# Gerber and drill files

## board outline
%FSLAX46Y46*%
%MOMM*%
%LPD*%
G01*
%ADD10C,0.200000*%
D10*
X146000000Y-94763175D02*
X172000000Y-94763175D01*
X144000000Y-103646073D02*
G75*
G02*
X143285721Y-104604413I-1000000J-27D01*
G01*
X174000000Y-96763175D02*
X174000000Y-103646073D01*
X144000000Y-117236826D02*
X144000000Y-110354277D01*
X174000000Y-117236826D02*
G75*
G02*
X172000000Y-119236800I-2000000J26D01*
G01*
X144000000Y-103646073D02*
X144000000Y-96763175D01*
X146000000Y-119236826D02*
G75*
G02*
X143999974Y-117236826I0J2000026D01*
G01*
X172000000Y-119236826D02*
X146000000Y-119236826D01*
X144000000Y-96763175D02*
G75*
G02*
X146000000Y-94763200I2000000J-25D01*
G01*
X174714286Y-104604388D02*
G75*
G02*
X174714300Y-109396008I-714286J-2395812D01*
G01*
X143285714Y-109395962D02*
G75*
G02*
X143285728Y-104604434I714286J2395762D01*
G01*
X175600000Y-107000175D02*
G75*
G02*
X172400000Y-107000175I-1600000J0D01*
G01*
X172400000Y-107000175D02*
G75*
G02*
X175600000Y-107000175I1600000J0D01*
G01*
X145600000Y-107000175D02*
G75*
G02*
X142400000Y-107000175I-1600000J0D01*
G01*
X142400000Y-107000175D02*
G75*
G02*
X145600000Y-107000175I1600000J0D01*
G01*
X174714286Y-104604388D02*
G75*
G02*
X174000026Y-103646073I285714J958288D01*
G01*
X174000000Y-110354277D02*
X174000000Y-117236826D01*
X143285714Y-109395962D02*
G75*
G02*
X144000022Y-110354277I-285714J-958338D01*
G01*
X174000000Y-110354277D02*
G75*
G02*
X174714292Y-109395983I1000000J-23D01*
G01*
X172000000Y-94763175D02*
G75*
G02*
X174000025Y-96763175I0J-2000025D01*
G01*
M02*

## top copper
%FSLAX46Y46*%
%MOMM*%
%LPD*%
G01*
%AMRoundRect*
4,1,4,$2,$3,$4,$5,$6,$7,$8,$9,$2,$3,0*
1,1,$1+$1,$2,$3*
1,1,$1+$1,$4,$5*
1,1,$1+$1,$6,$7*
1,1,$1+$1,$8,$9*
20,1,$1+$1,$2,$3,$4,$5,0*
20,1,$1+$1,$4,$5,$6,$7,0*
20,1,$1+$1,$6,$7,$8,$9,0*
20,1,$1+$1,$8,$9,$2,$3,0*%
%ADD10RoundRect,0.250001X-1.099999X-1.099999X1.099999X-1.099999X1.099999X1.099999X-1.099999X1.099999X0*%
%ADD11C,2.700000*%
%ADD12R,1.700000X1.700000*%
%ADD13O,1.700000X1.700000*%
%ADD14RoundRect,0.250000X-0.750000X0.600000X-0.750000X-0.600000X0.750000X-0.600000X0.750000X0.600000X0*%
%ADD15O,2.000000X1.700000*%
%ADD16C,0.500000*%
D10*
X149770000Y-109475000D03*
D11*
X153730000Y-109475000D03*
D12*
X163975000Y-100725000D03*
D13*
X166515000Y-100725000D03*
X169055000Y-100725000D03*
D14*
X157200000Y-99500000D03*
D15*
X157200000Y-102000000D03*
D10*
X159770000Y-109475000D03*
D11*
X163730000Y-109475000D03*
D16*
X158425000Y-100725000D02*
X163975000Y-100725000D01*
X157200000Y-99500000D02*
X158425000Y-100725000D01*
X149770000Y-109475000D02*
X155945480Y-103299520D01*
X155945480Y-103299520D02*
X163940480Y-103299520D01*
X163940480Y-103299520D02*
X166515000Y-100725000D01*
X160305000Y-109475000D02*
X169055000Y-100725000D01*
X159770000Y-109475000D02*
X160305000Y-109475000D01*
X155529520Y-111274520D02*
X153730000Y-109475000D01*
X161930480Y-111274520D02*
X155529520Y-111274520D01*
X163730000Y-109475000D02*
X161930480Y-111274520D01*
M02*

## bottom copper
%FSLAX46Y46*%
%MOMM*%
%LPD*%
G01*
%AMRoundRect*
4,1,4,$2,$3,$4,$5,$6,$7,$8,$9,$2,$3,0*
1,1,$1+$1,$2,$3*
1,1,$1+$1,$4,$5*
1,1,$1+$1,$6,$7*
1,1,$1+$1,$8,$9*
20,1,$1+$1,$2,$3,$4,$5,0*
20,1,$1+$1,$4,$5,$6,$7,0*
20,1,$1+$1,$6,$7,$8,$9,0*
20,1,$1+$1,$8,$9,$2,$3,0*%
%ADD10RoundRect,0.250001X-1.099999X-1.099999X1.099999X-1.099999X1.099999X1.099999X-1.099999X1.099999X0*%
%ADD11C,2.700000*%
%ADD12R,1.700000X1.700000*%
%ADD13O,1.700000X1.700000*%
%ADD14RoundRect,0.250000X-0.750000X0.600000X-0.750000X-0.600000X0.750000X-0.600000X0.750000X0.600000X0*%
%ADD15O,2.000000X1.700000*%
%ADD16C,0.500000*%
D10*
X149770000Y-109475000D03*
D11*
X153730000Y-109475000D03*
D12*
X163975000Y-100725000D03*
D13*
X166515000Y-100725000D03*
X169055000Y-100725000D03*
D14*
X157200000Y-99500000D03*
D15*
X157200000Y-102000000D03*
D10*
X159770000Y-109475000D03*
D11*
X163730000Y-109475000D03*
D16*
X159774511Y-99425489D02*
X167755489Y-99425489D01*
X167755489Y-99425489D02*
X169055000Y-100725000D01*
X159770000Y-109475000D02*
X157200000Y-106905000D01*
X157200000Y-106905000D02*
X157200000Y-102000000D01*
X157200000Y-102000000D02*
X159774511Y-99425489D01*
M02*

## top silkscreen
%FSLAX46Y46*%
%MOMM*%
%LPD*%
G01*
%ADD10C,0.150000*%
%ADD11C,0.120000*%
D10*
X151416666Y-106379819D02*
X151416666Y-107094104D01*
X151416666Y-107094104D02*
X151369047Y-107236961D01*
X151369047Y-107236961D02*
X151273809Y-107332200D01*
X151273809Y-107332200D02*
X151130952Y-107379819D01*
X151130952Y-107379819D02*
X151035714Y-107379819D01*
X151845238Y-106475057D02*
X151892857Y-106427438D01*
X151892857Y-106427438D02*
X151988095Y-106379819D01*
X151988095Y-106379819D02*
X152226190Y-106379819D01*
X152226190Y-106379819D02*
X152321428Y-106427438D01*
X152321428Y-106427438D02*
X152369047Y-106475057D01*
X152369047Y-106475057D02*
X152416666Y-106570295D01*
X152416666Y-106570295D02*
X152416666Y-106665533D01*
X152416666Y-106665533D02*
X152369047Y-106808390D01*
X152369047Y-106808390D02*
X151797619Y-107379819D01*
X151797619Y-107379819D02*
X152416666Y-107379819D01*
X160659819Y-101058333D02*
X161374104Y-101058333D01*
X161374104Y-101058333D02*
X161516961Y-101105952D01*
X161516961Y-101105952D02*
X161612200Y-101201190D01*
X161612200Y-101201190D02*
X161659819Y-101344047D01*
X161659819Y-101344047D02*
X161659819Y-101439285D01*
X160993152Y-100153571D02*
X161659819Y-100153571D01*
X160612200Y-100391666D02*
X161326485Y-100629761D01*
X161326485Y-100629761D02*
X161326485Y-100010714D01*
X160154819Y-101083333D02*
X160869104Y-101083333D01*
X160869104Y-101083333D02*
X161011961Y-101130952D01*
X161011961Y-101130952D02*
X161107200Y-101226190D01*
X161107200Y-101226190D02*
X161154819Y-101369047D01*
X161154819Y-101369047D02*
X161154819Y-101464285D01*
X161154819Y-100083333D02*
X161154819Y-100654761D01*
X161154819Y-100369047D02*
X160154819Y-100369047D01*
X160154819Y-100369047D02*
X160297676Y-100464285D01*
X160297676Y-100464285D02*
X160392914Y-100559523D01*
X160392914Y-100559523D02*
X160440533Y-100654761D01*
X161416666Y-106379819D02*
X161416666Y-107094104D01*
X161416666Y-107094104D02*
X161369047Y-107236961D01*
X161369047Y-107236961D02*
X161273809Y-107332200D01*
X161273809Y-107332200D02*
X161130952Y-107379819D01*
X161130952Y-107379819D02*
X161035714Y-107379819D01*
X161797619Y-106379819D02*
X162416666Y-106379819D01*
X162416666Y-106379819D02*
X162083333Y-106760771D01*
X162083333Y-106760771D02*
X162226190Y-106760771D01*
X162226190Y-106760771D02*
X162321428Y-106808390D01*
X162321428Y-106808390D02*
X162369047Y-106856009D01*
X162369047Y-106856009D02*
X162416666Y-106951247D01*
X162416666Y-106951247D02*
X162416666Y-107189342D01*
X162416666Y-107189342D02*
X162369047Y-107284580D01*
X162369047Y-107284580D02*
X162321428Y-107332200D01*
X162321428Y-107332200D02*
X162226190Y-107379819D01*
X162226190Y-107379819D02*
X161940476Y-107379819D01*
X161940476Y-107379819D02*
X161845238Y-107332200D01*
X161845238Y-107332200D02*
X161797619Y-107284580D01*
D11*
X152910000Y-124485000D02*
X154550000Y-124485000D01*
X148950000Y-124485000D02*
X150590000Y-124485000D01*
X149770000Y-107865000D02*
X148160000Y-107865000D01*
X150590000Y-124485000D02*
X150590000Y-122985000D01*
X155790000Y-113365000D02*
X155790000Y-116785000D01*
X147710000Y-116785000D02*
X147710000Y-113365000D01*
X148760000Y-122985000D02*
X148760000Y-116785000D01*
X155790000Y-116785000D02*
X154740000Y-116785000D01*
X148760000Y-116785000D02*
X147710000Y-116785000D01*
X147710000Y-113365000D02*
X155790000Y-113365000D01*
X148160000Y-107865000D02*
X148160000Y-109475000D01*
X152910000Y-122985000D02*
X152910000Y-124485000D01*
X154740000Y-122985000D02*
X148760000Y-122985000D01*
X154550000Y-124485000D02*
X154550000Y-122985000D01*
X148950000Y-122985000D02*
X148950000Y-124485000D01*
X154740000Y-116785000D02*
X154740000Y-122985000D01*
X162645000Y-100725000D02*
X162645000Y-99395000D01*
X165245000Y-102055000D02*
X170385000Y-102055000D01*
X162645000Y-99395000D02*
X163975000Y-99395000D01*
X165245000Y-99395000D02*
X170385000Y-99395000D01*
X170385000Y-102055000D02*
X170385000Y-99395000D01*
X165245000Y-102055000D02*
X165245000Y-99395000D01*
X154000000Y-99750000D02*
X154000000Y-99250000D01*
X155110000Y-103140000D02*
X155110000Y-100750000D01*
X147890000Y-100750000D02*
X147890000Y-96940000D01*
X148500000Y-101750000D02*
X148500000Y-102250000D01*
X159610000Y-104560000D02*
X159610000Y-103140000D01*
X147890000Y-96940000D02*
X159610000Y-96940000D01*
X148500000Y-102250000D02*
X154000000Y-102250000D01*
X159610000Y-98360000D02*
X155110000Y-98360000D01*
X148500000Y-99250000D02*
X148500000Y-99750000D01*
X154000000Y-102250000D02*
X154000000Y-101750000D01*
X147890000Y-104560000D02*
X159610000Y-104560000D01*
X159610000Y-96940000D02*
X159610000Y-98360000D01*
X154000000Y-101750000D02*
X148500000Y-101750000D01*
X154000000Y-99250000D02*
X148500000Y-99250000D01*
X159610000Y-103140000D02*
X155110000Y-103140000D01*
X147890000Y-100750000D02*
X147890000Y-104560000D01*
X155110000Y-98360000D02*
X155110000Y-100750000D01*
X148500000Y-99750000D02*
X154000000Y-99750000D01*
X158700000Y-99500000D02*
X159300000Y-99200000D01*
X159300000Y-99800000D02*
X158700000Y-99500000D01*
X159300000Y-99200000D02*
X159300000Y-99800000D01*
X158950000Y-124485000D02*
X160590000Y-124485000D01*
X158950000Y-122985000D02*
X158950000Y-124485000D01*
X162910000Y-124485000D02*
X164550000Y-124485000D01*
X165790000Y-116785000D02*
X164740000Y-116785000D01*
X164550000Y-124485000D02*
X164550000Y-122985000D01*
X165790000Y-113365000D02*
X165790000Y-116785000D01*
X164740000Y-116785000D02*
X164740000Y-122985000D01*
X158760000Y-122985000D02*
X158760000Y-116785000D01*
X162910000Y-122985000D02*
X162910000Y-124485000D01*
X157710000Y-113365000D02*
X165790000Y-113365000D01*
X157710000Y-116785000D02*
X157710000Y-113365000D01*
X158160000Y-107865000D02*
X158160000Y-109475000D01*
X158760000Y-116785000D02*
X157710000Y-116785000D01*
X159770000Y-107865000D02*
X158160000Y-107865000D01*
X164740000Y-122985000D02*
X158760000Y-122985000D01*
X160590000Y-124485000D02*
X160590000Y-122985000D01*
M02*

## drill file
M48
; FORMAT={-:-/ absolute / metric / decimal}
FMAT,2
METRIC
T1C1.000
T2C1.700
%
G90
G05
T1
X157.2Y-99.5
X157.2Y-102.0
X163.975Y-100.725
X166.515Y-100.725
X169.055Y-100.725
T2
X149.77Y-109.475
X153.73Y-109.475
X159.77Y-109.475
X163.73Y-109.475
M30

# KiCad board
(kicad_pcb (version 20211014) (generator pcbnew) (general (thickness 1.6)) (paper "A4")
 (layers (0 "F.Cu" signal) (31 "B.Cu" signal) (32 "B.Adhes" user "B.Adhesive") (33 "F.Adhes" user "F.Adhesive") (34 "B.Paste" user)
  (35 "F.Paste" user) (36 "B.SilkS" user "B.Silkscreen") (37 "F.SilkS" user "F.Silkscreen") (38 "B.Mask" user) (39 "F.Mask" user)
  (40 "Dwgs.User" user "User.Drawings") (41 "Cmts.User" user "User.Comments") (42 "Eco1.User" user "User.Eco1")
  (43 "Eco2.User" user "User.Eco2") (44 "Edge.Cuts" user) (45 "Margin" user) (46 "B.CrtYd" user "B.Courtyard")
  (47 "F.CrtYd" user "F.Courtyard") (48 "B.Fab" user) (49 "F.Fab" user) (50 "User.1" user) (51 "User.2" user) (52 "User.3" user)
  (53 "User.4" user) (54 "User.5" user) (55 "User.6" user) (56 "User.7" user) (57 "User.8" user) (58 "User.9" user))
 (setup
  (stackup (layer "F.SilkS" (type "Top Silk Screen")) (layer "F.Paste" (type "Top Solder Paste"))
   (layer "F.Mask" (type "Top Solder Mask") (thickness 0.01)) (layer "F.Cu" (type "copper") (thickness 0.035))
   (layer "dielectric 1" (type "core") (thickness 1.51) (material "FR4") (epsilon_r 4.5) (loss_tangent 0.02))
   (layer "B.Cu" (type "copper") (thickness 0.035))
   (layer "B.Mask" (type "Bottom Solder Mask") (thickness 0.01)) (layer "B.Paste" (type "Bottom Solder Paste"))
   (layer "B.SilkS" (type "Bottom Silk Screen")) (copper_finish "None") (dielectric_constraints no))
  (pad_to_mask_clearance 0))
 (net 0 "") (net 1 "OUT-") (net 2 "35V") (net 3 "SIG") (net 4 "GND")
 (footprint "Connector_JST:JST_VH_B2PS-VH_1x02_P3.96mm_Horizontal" (layer "F.Cu") (at 149.77 109.475)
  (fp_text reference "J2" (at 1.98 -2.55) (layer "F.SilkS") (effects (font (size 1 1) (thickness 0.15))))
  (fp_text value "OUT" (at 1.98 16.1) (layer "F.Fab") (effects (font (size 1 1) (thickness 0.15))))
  (fp_line (start 3.14 15.01) (end 4.78 15.01) (layer "F.SilkS") (width 0.12))
  (fp_line (start -0.82 15.01) (end 0.82 15.01) (layer "F.SilkS") (width 0.12))
  (fp_line (start 0 -1.61) (end -1.61 -1.61) (layer "F.SilkS") (width 0.12))
  (fp_line (start 0.82 15.01) (end 0.82 13.51) (layer "F.SilkS") (width 0.12))
  (fp_line (start 6.02 3.89) (end 6.02 7.31) (layer "F.SilkS") (width 0.12))
  (fp_line (start -2.06 7.31) (end -2.06 3.89) (layer "F.SilkS") (width 0.12))
  (fp_line (start -1.01 13.51) (end -1.01 7.31) (layer "F.SilkS") (width 0.12))
  (fp_line (start 6.02 7.31) (end 4.97 7.31) (layer "F.SilkS") (width 0.12))
  (fp_line (start -1.01 7.31) (end -2.06 7.31) (layer "F.SilkS") (width 0.12))
  (fp_line (start -2.06 3.89) (end 6.02 3.89) (layer "F.SilkS") (width 0.12))
  (fp_line (start -1.61 -1.61) (end -1.61 0) (layer "F.SilkS") (width 0.12))
  (fp_line (start 3.14 13.51) (end 3.14 15.01) (layer "F.SilkS") (width 0.12))
  (fp_line (start 4.97 13.51) (end -1.01 13.51) (layer "F.SilkS") (width 0.12))
  (fp_line (start 4.78 15.01) (end 4.78 13.51) (layer "F.SilkS") (width 0.12))
  (fp_line (start -0.82 13.51) (end -0.82 15.01) (layer "F.SilkS") (width 0.12))
  (fp_line (start 4.97 7.31) (end 4.97 13.51) (layer "F.SilkS") (width 0.12))
  (pad "1" thru_hole roundrect (at 0 0) (size 2.7 2.7) (drill 1.7) (layers *.Cu *.Mask) (roundrect_rratio 0.09259296296) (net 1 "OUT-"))
  (pad "2" thru_hole circle (at 3.96 0) (size 2.7 2.7) (drill 1.7) (layers *.Cu *.Mask) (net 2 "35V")))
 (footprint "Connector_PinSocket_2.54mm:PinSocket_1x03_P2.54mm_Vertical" (layer "F.Cu") (at 163.975 100.725 90)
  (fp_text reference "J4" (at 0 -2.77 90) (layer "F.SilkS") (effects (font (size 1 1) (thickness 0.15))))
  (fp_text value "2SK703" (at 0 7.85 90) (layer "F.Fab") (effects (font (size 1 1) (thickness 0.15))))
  (fp_line (start 0 -1.33) (end 1.33 -1.33) (layer "F.SilkS") (width 0.12))
  (fp_line (start -1.33 1.27) (end -1.33 6.41) (layer "F.SilkS") (width 0.12))
  (fp_line (start 1.33 -1.33) (end 1.33 0) (layer "F.SilkS") (width 0.12))
  (fp_line (start 1.33 1.27) (end 1.33 6.41) (layer "F.SilkS") (width 0.12))
  (fp_line (start -1.33 6.41) (end 1.33 6.41) (layer "F.SilkS") (width 0.12))
  (fp_line (start -1.33 1.27) (end 1.33 1.27) (layer "F.SilkS") (width 0.12))
  (pad "1" thru_hole rect (at 0 0 90) (size 1.7 1.7) (drill 1) (layers *.Cu *.Mask) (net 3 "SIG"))
  (pad "2" thru_hole oval (at 0 2.54 90) (size 1.7 1.7) (drill 1) (layers *.Cu *.Mask) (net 1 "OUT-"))
  (pad "3" thru_hole oval (at 0 5.08 90) (size 1.7 1.7) (drill 1) (layers *.Cu *.Mask) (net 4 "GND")))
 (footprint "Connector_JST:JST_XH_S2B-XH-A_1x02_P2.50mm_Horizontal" (layer "F.Cu") (at 157.2 99.5 -90)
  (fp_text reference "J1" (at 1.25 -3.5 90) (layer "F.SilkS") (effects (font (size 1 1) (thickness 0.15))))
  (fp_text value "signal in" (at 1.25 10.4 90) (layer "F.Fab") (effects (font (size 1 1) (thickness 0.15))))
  (fp_line (start 0.25 3.2) (end -0.25 3.2) (layer "F.SilkS") (width 0.12))
  (fp_line (start 3.64 2.09) (end 1.25 2.09) (layer "F.SilkS") (width 0.12))
  (fp_line (start 1.25 9.31) (end -2.56 9.31) (layer "F.SilkS") (width 0.12))
  (fp_line (start 2.25 8.7) (end 2.75 8.7) (layer "F.SilkS") (width 0.12))
  (fp_line (start 5.06 -2.41) (end 3.64 -2.41) (layer "F.SilkS") (width 0.12))
  (fp_line (start -2.56 9.31) (end -2.56 -2.41) (layer "F.SilkS") (width 0.12))
  (fp_line (start 2.75 8.7) (end 2.75 3.2) (layer "F.SilkS") (width 0.12))
  (fp_line (start -1.14 -2.41) (end -1.14 2.09) (layer "F.SilkS") (width 0.12))
  (fp_line (start -0.25 8.7) (end 0.25 8.7) (layer "F.SilkS") (width 0.12))
  (fp_line (start 2.75 3.2) (end 2.25 3.2) (layer "F.SilkS") (width 0.12))
  (fp_line (start 5.06 9.31) (end 5.06 -2.41) (layer "F.SilkS") (width 0.12))
  (fp_line (start -2.56 -2.41) (end -1.14 -2.41) (layer "F.SilkS") (width 0.12))
  (fp_line (start 2.25 3.2) (end 2.25 8.7) (layer "F.SilkS") (width 0.12))
  (fp_line (start -0.25 3.2) (end -0.25 8.7) (layer "F.SilkS") (width 0.12))
  (fp_line (start 3.64 -2.41) (end 3.64 2.09) (layer "F.SilkS") (width 0.12))
  (fp_line (start 1.25 9.31) (end 5.06 9.31) (layer "F.SilkS") (width 0.12))
  (fp_line (start -1.14 2.09) (end 1.25 2.09) (layer "F.SilkS") (width 0.12))
  (fp_line (start 0.25 8.7) (end 0.25 3.2) (layer "F.SilkS") (width 0.12))
  (fp_line (start 0 -1.5) (end -0.3 -2.1) (layer "F.SilkS") (width 0.12))
  (fp_line (start 0.3 -2.1) (end 0 -1.5) (layer "F.SilkS") (width 0.12))
  (fp_line (start -0.3 -2.1) (end 0.3 -2.1) (layer "F.SilkS") (width 0.12))
  (pad "1" thru_hole roundrect (at 0 0 270) (size 1.7 2) (drill 1) (layers *.Cu *.Mask) (roundrect_rratio 0.1470588235) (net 3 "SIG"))
  (pad "2" thru_hole oval (at 2.5 0 270) (size 1.7 2) (drill 1) (layers *.Cu *.Mask) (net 4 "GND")))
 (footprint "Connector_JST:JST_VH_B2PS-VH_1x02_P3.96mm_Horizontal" (layer "F.Cu") (at 159.77 109.475)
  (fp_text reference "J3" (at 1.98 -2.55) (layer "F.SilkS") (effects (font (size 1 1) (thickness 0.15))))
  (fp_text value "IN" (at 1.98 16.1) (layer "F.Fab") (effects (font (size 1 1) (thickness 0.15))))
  (fp_line (start -0.82 15.01) (end 0.82 15.01) (layer "F.SilkS") (width 0.12))
  (fp_line (start -0.82 13.51) (end -0.82 15.01) (layer "F.SilkS") (width 0.12))
  (fp_line (start 3.14 15.01) (end 4.78 15.01) (layer "F.SilkS") (width 0.12))
  (fp_line (start 6.02 7.31) (end 4.97 7.31) (layer "F.SilkS") (width 0.12))
  (fp_line (start 4.78 15.01) (end 4.78 13.51) (layer "F.SilkS") (width 0.12))
  (fp_line (start 6.02 3.89) (end 6.02 7.31) (layer "F.SilkS") (width 0.12))
  (fp_line (start 4.97 7.31) (end 4.97 13.51) (layer "F.SilkS") (width 0.12))
  (fp_line (start -1.01 13.51) (end -1.01 7.31) (layer "F.SilkS") (width 0.12))
  (fp_line (start 3.14 13.51) (end 3.14 15.01) (layer "F.SilkS") (width 0.12))
  (fp_line (start -2.06 3.89) (end 6.02 3.89) (layer "F.SilkS") (width 0.12))
  (fp_line (start -2.06 7.31) (end -2.06 3.89) (layer "F.SilkS") (width 0.12))
  (fp_line (start -1.61 -1.61) (end -1.61 0) (layer "F.SilkS") (width 0.12))
  (fp_line (start -1.01 7.31) (end -2.06 7.31) (layer "F.SilkS") (width 0.12))
  (fp_line (start 0 -1.61) (end -1.61 -1.61) (layer "F.SilkS") (width 0.12))
  (fp_line (start 4.97 13.51) (end -1.01 13.51) (layer "F.SilkS") (width 0.12))
  (fp_line (start 0.82 15.01) (end 0.82 13.51) (layer "F.SilkS") (width 0.12))
  (pad "1" thru_hole roundrect (at 0 0) (size 2.7 2.7) (drill 1.7) (layers *.Cu *.Mask) (roundrect_rratio 0.09259296296) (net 4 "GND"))
  (pad "2" thru_hole circle (at 3.96 0) (size 2.7 2.7) (drill 1.7) (layers *.Cu *.Mask) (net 2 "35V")))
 (gr_line (start 146 94.763175) (end 172 94.763175) (layer "Edge.Cuts") (width 0.2))
 (gr_arc (start 144 103.646073) (mid 143.801784 104.243688) (end 143.285714 104.604388) (layer "Edge.Cuts") (width 0.2))
 (gr_line (start 174 96.763175) (end 174 103.646073) (layer "Edge.Cuts") (width 0.2))
 (gr_line (start 144 117.236826) (end 144 110.354277) (layer "Edge.Cuts") (width 0.2))
 (gr_arc (start 174 117.236826) (mid 173.414214 118.65104) (end 172 119.236826) (layer "Edge.Cuts") (width 0.2))
 (gr_line (start 144 103.646073) (end 144 96.763175) (layer "Edge.Cuts") (width 0.2))
 (gr_arc (start 146 119.236826) (mid 144.585786 118.65104) (end 144 117.236826) (layer "Edge.Cuts") (width 0.2))
 (gr_line (start 172 119.236826) (end 146 119.236826) (layer "Edge.Cuts") (width 0.2))
 (gr_arc (start 144 96.763175) (mid 144.585786 95.348961) (end 146 94.763175) (layer "Edge.Cuts") (width 0.2))
 (gr_arc (start 174.714286 104.604388) (mid 176.5 107.000175) (end 174.714286 109.395962) (layer "Edge.Cuts") (width 0.2))
 (gr_arc (start 143.285714 109.395962) (mid 141.5 107.000175) (end 143.285714 104.604388) (layer "Edge.Cuts") (width 0.2))
 (gr_circle (center 174 107.000175) (end 174 105.400175) (layer "Edge.Cuts") (width 0.2) (fill none))
 (gr_circle (center 144 107.000175) (end 144 105.400175) (layer "Edge.Cuts") (width 0.2) (fill none))
 (gr_arc (start 174.714286 104.604388) (mid 174.198216 104.243688) (end 174 103.646073) (layer "Edge.Cuts") (width 0.2))
 (gr_line (start 174 110.354277) (end 174 117.236826) (layer "Edge.Cuts") (width 0.2))
 (gr_arc (start 143.285714 109.395962) (mid 143.801784 109.756663) (end 144 110.354277) (layer "Edge.Cuts") (width 0.2))
 (gr_arc (start 174 110.354277) (mid 174.198216 109.756663) (end 174.714286 109.395962) (layer "Edge.Cuts") (width 0.2))
 (gr_arc (start 172 94.763175) (mid 173.414214 95.348961) (end 174 96.763175) (layer "Edge.Cuts") (width 0.2))
 (segment (start 158.425 100.725) (end 163.975 100.725) (width 0.5) (layer "F.Cu") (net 3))
 (segment (start 157.2 99.5) (end 158.425 100.725) (width 0.5) (layer "F.Cu") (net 3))
 (segment (start 149.77 109.475) (end 155.94548 103.29952) (width 0.5) (layer "F.Cu") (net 1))
 (segment (start 155.94548 103.29952) (end 163.94048 103.29952) (width 0.5) (layer "F.Cu") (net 1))
 (segment (start 163.94048 103.29952) (end 166.515 100.725) (width 0.5) (layer "F.Cu") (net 1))
 (segment (start 160.305 109.475) (end 169.055 100.725) (width 0.5) (layer "F.Cu") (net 4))
 (segment (start 159.77 109.475) (end 160.305 109.475) (width 0.5) (layer "F.Cu") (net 4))
 (segment (start 159.774511 99.425489) (end 167.755489 99.425489) (width 0.5) (layer "B.Cu") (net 4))
 (segment (start 167.755489 99.425489) (end 169.055 100.725) (width 0.5) (layer "B.Cu") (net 4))
 (segment (start 159.77 109.475) (end 157.2 106.905) (width 0.5) (layer "B.Cu") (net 4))
 (segment (start 157.2 106.905) (end 157.2 102) (width 0.5) (layer "B.Cu") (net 4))
 (segment (start 157.2 102) (end 159.774511 99.425489) (width 0.5) (layer "B.Cu") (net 4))
 (segment (start 155.52952 111.27452) (end 153.73 109.475) (width 0.5) (layer "F.Cu") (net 2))
 (segment (start 161.93048 111.27452) (end 155.52952 111.27452) (width 0.5) (layer "F.Cu") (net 2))
 (segment (start 163.73 109.475) (end 161.93048 111.27452) (width 0.5) (layer "F.Cu") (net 2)))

